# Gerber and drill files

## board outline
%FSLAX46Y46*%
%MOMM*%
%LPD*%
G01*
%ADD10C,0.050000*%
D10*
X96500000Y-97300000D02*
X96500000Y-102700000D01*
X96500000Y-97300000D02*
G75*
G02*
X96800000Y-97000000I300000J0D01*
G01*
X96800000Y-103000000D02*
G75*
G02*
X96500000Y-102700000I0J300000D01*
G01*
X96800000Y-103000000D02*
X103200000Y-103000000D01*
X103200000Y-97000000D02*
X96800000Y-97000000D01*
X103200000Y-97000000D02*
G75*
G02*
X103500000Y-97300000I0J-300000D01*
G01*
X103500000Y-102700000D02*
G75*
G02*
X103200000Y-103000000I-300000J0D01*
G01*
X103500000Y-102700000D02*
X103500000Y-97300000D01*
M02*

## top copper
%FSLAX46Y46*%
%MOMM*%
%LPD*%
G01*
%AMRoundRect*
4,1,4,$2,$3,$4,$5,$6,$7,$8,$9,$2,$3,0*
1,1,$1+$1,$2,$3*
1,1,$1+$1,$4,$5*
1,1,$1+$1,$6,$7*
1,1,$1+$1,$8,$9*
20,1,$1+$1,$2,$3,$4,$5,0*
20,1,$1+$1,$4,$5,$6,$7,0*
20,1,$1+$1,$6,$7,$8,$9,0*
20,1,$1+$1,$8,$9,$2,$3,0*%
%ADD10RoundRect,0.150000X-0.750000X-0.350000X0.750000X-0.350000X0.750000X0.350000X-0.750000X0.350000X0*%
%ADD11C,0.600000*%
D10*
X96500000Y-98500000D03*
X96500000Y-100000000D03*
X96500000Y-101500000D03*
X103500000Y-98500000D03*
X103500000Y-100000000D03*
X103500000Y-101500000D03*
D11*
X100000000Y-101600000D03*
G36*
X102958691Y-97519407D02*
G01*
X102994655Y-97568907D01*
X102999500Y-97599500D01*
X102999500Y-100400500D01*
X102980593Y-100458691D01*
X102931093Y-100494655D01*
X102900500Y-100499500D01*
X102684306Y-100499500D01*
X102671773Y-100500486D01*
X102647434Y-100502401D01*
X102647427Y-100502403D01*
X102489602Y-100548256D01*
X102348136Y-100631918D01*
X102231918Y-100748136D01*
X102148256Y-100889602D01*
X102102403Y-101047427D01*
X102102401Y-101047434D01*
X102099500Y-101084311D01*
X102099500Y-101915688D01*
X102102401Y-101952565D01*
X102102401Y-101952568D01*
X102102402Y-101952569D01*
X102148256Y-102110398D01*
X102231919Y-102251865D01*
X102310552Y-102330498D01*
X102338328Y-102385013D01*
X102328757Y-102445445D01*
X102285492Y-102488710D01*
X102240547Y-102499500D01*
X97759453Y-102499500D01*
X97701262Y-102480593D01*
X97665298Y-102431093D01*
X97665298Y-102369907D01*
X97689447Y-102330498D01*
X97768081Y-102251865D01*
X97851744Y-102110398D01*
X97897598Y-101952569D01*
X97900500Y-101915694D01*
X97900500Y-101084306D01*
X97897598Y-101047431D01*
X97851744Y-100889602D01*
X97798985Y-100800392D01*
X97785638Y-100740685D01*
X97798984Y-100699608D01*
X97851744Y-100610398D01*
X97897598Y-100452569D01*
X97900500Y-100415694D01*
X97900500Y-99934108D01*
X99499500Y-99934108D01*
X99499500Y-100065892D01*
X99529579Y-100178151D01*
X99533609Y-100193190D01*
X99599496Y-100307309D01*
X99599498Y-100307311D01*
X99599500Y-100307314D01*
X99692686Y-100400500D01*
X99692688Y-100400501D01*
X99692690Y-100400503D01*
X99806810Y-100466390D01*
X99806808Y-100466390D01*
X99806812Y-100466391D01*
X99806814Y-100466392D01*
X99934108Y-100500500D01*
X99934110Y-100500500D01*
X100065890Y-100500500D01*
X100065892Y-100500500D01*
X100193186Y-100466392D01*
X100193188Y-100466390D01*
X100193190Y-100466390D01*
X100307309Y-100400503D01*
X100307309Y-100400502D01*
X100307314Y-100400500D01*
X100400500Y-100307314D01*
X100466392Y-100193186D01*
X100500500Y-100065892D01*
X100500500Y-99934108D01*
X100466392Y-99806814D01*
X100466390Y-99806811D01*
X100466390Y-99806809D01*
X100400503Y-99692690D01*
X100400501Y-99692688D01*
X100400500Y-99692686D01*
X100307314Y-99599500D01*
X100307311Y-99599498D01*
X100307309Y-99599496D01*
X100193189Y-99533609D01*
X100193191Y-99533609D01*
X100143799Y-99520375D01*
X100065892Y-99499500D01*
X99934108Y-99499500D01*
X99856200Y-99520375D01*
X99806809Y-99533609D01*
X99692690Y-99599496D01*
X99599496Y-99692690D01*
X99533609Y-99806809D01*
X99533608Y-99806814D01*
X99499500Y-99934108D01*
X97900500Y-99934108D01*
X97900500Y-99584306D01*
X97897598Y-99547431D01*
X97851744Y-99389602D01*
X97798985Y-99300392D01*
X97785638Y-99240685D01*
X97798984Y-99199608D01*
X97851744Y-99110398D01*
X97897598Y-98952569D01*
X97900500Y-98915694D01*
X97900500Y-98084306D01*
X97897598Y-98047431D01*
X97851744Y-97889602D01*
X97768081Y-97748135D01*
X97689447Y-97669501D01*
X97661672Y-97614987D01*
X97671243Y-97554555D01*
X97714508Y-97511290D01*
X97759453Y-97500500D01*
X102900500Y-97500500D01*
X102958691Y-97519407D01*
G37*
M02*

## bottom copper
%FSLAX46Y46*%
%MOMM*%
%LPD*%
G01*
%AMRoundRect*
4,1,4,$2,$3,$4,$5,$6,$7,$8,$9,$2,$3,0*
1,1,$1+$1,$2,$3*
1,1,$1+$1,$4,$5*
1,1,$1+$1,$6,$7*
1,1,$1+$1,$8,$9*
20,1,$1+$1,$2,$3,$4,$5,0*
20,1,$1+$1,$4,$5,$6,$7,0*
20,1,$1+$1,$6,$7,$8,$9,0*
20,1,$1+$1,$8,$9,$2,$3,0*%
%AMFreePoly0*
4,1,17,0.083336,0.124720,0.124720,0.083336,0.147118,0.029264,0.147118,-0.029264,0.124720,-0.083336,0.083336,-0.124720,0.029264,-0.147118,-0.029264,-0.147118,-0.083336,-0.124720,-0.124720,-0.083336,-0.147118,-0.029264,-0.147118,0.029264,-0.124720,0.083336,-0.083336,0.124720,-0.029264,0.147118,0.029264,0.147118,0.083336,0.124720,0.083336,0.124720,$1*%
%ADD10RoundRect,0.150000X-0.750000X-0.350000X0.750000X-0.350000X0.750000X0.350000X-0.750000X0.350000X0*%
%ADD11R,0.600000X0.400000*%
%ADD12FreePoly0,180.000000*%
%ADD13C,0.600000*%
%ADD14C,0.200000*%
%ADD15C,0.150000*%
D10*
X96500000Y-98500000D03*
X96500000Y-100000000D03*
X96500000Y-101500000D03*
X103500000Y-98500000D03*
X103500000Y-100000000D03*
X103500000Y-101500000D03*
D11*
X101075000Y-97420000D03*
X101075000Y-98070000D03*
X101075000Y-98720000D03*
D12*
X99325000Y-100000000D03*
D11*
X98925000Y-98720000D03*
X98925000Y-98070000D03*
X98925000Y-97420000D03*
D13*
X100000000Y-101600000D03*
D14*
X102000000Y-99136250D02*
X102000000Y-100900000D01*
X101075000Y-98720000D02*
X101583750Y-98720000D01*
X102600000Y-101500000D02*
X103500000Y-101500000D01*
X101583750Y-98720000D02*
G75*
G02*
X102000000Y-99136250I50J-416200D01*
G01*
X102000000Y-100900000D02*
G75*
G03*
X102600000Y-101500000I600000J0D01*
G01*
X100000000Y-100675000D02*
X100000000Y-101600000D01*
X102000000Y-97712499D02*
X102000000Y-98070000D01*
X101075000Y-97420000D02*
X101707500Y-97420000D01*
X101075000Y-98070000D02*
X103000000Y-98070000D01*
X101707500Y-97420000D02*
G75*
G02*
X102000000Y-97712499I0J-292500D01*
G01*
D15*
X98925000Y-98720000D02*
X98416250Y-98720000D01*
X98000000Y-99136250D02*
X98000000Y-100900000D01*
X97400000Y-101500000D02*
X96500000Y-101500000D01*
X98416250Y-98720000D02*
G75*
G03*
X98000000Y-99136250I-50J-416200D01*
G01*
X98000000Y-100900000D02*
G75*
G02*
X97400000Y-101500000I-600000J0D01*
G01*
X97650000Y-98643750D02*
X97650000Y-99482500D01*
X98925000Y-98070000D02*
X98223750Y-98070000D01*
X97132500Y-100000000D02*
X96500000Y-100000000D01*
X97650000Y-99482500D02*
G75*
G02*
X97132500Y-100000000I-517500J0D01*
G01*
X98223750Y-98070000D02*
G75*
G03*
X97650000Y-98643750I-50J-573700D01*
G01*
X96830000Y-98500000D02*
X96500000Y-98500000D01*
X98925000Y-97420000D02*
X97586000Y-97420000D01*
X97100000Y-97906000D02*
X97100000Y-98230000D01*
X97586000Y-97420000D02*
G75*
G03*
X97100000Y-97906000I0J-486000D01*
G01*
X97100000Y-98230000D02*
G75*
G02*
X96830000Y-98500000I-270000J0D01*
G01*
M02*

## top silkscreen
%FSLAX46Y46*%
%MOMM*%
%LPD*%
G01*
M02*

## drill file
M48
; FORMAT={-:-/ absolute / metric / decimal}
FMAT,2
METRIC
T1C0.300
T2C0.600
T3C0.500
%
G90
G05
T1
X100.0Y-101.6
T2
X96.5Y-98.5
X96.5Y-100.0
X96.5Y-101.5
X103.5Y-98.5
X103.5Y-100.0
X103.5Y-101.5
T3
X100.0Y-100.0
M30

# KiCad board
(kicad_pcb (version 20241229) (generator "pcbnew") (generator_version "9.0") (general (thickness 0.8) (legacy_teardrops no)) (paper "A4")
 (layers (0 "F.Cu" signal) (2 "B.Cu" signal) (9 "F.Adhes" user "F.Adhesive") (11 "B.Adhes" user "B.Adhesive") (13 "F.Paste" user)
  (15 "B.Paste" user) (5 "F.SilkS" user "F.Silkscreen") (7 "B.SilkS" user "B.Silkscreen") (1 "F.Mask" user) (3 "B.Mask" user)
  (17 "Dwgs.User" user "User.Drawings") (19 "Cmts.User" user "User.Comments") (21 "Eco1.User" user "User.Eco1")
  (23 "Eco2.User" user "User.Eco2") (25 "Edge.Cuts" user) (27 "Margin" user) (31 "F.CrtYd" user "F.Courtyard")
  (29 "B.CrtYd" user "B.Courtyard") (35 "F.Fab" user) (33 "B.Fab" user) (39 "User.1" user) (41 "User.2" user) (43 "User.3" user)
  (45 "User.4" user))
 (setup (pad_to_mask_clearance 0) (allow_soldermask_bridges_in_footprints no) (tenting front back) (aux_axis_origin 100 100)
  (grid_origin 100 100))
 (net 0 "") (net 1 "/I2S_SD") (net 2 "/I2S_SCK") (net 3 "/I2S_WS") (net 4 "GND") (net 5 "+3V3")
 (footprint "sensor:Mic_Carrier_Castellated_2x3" (layer "F.Cu") (at 100 100)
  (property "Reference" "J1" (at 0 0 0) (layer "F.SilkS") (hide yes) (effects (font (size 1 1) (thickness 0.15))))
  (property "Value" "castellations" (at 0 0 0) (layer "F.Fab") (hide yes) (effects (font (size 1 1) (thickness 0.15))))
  (pad "1" thru_hole roundrect (at -3.5 -1.5) (size 1.8 1) (drill 0.6) (layers "*.Cu" "*.Mask") (remove_unused_layers no)
   (roundrect_rratio 0.15) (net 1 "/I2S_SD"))
  (pad "2" thru_hole roundrect (at -3.5 0) (size 1.8 1) (drill 0.6) (layers "*.Cu" "*.Mask") (remove_unused_layers no)
   (roundrect_rratio 0.15) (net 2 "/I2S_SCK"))
  (pad "3" thru_hole roundrect (at -3.5 1.5) (size 1.8 1) (drill 0.6) (layers "*.Cu" "*.Mask") (remove_unused_layers no)
   (roundrect_rratio 0.15) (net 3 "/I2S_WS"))
  (pad "4" thru_hole roundrect (at 3.5 -1.5) (size 1.8 1) (drill 0.6) (layers "*.Cu" "*.Mask") (remove_unused_layers no)
   (roundrect_rratio 0.15) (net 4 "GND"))
  (pad "5" thru_hole roundrect (at 3.5 0) (size 1.8 1) (drill 0.6) (layers "*.Cu" "*.Mask") (remove_unused_layers no)
   (roundrect_rratio 0.15) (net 4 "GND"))
  (pad "6" thru_hole roundrect (at 3.5 1.5) (size 1.8 1) (drill 0.6) (layers "*.Cu" "*.Mask") (remove_unused_layers no)
   (roundrect_rratio 0.15) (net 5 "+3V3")))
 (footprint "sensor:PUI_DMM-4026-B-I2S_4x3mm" (layer "B.Cu") (at 100 99 180)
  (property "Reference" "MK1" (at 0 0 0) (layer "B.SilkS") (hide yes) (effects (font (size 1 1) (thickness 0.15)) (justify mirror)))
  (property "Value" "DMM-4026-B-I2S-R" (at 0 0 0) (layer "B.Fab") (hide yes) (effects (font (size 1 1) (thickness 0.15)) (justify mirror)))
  (pad "" np_thru_hole circle (at 0 -1 180) (size 0.5 0.5) (drill 0.5) (layers "*.Mask"))
  (pad "1" smd rect (at -1.075 1.58 180) (size 0.6 0.4) (layers "B.Cu" "B.Mask" "B.Paste") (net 4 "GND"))
  (pad "2" smd rect (at -1.075 0.93 180) (size 0.6 0.4) (layers "B.Cu" "B.Mask" "B.Paste") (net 4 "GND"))
  (pad "3" smd rect (at -1.075 0.28 180) (size 0.6 0.4) (layers "B.Cu" "B.Mask" "B.Paste") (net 5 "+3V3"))
  (pad "4" smd custom (at 0.675 -1 180) (size 0.3 0.3) (layers "B.Cu" "B.Mask" "B.Paste") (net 4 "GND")
   (options (clearance outline) (anchor circle)) (primitives))
  (pad "5" smd rect (at 1.075 0.28 180) (size 0.6 0.4) (layers "B.Cu" "B.Mask" "B.Paste") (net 3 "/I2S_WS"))
  (pad "6" smd rect (at 1.075 0.93 180) (size 0.6 0.4) (layers "B.Cu" "B.Mask" "B.Paste") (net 2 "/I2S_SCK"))
  (pad "7" smd rect (at 1.075 1.58 180) (size 0.6 0.4) (layers "B.Cu" "B.Mask" "B.Paste") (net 1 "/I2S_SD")))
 (gr_line (start 96.5 97.3) (end 96.5 102.7) (stroke (width 0.05) (type default)) (layer "Edge.Cuts"))
 (gr_arc (start 96.5 97.3) (mid 96.587868 97.087868) (end 96.8 97) (stroke (width 0.05) (type default)) (layer "Edge.Cuts"))
 (gr_arc (start 96.8 103) (mid 96.587868 102.912132) (end 96.5 102.7) (stroke (width 0.05) (type default)) (layer "Edge.Cuts"))
 (gr_line (start 96.8 103) (end 103.2 103) (stroke (width 0.05) (type default)) (layer "Edge.Cuts"))
 (gr_line (start 103.2 97) (end 96.8 97) (stroke (width 0.05) (type default)) (layer "Edge.Cuts"))
 (gr_arc (start 103.2 97) (mid 103.412132 97.087868) (end 103.5 97.3) (stroke (width 0.05) (type default)) (layer "Edge.Cuts"))
 (gr_arc (start 103.5 102.7) (mid 103.412132 102.912132) (end 103.2 103) (stroke (width 0.05) (type default)) (layer "Edge.Cuts"))
 (gr_line (start 103.5 102.7) (end 103.5 97.3) (stroke (width 0.05) (type default)) (layer "Edge.Cuts"))
 (segment (start 102 99.13625) (end 102 100.9) (width 0.2) (layer "B.Cu") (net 5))
 (segment (start 101.075 98.72) (end 101.58375 98.72) (width 0.2) (layer "B.Cu") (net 5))
 (segment (start 102.6 101.5) (end 103.5 101.5) (width 0.2) (layer "B.Cu") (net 5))
 (arc (start 101.58375 98.72) (mid 101.878083 98.841916) (end 102 99.13625) (width 0.2) (layer "B.Cu") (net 5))
 (arc (start 102 100.9) (mid 102.175735 101.324264) (end 102.6 101.5) (width 0.2) (layer "B.Cu") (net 5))
 (via (at 100 101.6) (size 0.6) (drill 0.3) (layers "F.Cu" "B.Cu") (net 4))
 (segment (start 100 100.675) (end 100 101.6) (width 0.2) (layer "B.Cu") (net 4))
 (segment (start 102 97.712499) (end 102 98.07) (width 0.2) (layer "B.Cu") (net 4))
 (segment (start 101.075 97.42) (end 101.7075 97.42) (width 0.2) (layer "B.Cu") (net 4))
 (segment (start 101.075 98.07) (end 103 98.07) (width 0.2) (layer "B.Cu") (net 4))
 (arc (start 101.7075 97.42) (mid 101.914328 97.505671) (end 102 97.712499) (width 0.2) (layer "B.Cu") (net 4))
 (segment (start 98.925 98.72) (end 98.41625 98.72) (width 0.15) (layer "B.Cu") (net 3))
 (segment (start 98 99.13625) (end 98 100.9) (width 0.15) (layer "B.Cu") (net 3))
 (segment (start 97.4 101.5) (end 96.5 101.5) (width 0.15) (layer "B.Cu") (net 3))
 (arc (start 98.41625 98.72) (mid 98.121916 98.841916) (end 98 99.13625) (width 0.15) (layer "B.Cu") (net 3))
 (arc (start 98 100.9) (mid 97.824264 101.324264) (end 97.4 101.5) (width 0.15) (layer "B.Cu") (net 3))
 (segment (start 97.65 98.64375) (end 97.65 99.4825) (width 0.15) (layer "B.Cu") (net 2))
 (segment (start 98.925 98.07) (end 98.22375 98.07) (width 0.15) (layer "B.Cu") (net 2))
 (segment (start 97.1325 100) (end 96.5 100) (width 0.15) (layer "B.Cu") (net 2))
 (arc (start 97.65 99.4825) (mid 97.498427 99.848427) (end 97.1325 100) (width 0.15) (layer "B.Cu") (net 2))
 (arc (start 98.22375 98.07) (mid 97.818047 98.238047) (end 97.65 98.64375) (width 0.15) (layer "B.Cu") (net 2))
 (segment (start 96.83 98.5) (end 96.5 98.5) (width 0.15) (layer "B.Cu") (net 1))
 (segment (start 98.925 97.42) (end 97.586 97.42) (width 0.15) (layer "B.Cu") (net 1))
 (segment (start 97.1 97.906) (end 97.1 98.23) (width 0.15) (layer "B.Cu") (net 1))
 (arc (start 97.586 97.42) (mid 97.242346 97.562346) (end 97.1 97.906) (width 0.15) (layer "B.Cu") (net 1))
 (arc (start 97.1 98.23) (mid 97.020918 98.420918) (end 96.83 98.5) (width 0.15) (layer "B.Cu") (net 1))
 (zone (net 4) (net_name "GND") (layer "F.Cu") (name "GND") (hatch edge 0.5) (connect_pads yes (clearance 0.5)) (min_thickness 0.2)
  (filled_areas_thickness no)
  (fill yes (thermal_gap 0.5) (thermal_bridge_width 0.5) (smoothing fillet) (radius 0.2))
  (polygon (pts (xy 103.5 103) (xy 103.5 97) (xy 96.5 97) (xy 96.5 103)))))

